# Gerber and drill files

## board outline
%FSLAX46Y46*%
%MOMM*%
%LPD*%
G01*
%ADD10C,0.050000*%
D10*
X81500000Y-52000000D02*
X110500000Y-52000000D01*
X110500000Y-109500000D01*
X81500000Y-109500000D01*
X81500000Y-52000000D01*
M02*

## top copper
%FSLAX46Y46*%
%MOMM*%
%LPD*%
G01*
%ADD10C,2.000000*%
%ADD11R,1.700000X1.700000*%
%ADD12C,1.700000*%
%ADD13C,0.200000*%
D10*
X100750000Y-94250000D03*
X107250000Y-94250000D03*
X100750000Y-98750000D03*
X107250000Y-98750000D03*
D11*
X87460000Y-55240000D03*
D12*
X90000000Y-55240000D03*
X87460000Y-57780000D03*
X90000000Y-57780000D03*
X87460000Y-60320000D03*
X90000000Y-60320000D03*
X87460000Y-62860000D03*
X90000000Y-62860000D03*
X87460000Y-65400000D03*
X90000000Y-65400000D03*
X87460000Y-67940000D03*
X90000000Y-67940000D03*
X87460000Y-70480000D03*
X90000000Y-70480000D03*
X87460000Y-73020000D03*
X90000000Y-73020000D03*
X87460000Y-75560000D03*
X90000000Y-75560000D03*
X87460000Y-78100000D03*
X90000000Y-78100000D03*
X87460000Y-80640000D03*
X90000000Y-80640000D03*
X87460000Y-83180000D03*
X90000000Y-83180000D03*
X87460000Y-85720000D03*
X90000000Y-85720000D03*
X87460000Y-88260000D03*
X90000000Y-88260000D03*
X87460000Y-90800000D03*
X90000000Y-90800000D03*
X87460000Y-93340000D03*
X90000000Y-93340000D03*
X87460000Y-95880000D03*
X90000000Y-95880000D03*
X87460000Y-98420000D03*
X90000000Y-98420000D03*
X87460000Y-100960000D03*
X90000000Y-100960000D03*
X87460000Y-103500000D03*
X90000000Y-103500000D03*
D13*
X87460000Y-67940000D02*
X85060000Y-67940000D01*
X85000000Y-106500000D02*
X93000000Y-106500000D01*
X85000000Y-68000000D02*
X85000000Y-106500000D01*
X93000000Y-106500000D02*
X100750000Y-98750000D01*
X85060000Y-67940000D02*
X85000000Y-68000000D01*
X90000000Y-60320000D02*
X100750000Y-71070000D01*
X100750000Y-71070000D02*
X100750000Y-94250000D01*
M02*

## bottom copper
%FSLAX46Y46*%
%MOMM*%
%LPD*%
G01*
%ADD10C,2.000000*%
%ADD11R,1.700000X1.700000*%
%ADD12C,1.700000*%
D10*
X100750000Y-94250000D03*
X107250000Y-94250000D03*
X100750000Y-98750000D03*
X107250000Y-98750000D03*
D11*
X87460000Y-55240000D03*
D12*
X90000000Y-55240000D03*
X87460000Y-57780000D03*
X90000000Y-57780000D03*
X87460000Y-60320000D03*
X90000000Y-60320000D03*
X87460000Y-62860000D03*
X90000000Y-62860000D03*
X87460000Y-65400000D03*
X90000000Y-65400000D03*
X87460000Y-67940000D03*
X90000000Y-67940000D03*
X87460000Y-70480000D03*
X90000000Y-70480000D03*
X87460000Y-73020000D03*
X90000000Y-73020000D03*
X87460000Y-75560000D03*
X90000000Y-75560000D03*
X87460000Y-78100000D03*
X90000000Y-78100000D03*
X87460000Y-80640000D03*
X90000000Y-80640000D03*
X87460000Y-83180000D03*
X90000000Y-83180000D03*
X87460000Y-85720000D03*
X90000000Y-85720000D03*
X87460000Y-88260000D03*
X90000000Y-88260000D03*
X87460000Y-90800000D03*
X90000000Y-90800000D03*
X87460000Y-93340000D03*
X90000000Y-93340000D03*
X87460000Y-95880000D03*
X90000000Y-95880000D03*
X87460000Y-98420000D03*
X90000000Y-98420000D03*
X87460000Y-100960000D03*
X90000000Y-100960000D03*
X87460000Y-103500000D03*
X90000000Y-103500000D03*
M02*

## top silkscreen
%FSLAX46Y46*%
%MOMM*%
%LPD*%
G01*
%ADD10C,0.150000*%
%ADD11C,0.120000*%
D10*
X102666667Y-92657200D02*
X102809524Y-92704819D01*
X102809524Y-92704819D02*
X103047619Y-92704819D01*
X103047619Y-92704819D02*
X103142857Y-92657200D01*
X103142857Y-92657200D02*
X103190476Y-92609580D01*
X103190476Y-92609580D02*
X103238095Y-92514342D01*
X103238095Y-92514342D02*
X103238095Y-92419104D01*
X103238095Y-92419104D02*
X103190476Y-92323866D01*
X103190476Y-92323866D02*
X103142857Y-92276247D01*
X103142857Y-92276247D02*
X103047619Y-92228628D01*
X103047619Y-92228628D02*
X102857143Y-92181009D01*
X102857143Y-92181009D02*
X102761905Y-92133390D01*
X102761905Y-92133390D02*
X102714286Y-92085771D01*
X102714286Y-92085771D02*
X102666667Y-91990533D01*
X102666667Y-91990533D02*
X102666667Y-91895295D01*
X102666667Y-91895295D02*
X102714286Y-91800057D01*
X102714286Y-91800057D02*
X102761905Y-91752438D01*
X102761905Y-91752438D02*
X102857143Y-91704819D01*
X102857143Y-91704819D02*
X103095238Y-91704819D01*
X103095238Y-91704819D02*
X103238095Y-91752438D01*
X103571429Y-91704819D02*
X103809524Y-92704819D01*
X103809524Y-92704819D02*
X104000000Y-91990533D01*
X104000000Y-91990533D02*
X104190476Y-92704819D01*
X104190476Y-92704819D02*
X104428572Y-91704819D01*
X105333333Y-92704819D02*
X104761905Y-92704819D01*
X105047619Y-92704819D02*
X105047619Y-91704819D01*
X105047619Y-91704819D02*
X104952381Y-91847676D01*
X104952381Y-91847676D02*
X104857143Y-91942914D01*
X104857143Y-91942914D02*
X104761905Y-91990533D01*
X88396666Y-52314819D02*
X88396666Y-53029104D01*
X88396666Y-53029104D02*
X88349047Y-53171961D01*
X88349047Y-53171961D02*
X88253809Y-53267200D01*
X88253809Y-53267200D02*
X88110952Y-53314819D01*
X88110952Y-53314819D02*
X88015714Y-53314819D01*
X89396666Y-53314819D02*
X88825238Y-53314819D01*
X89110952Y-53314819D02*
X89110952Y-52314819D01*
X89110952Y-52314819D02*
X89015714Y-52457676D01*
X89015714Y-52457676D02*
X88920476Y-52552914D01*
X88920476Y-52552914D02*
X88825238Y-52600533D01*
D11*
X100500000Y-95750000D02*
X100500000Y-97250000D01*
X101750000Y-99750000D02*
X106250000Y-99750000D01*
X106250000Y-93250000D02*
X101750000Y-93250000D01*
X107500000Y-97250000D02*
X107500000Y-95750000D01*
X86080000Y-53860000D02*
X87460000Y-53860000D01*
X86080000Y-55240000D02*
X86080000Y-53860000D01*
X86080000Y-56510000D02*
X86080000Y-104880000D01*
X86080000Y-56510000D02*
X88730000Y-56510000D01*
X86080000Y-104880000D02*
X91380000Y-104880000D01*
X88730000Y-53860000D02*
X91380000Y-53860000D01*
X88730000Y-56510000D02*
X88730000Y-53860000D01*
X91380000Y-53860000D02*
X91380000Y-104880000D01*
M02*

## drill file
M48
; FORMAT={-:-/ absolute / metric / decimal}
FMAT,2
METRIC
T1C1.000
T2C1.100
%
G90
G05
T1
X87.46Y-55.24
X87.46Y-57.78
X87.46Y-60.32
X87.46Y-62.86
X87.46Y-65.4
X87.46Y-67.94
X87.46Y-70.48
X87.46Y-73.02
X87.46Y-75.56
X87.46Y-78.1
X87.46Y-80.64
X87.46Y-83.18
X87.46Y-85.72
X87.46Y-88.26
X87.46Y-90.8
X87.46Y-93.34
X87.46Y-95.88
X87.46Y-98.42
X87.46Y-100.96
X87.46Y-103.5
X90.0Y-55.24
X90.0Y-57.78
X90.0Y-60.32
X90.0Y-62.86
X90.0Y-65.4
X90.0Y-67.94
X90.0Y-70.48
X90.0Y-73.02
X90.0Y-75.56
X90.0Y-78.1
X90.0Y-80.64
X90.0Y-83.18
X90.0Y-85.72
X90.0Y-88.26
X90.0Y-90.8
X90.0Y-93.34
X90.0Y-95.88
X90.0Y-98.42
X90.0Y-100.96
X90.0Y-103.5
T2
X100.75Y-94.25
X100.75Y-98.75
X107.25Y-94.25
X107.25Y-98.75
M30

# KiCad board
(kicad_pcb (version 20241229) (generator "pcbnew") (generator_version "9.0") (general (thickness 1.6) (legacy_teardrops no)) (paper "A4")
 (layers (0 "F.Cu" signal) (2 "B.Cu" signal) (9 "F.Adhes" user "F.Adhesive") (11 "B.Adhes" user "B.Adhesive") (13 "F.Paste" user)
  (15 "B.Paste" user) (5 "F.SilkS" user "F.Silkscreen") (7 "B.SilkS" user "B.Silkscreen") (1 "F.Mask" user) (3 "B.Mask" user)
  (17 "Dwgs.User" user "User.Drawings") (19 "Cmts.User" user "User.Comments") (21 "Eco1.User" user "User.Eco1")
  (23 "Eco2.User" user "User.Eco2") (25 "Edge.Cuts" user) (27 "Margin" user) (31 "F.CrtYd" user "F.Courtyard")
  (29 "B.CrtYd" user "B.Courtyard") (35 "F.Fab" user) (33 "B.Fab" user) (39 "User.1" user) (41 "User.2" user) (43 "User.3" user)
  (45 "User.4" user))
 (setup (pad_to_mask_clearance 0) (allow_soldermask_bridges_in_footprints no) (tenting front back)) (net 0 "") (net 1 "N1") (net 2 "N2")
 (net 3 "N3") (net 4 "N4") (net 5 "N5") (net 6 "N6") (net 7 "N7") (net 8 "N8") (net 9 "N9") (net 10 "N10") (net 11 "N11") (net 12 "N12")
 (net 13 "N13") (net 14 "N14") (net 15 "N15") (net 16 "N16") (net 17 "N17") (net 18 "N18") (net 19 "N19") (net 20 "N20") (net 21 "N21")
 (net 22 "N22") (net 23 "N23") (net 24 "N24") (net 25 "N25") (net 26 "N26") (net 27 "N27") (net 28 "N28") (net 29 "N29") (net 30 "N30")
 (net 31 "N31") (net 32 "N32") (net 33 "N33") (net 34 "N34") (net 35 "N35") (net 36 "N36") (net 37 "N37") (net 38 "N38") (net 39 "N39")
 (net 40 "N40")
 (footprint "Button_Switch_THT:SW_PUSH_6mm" (layer "F.Cu") (at 100.75 94.25)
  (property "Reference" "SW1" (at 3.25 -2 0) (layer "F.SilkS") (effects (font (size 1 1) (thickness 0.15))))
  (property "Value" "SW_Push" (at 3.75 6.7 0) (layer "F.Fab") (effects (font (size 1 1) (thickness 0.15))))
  (fp_line (start -0.25 1.5) (end -0.25 3) (stroke (width 0.12) (type solid)) (layer "F.SilkS"))
  (fp_line (start 1 5.5) (end 5.5 5.5) (stroke (width 0.12) (type solid)) (layer "F.SilkS"))
  (fp_line (start 5.5 -1) (end 1 -1) (stroke (width 0.12) (type solid)) (layer "F.SilkS"))
  (fp_line (start 6.75 3) (end 6.75 1.5) (stroke (width 0.12) (type solid)) (layer "F.SilkS"))
  (pad "1" thru_hole circle (at 0 0 90) (size 2 2) (drill 1.1) (layers "*.Cu" "*.Mask") (remove_unused_layers no) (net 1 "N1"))
  (pad "1" thru_hole circle (at 6.5 0 90) (size 2 2) (drill 1.1) (layers "*.Cu" "*.Mask") (remove_unused_layers no) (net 1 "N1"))
  (pad "2" thru_hole circle (at 0 4.5 90) (size 2 2) (drill 1.1) (layers "*.Cu" "*.Mask") (remove_unused_layers no) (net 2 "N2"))
  (pad "2" thru_hole circle (at 6.5 4.5 90) (size 2 2) (drill 1.1) (layers "*.Cu" "*.Mask") (remove_unused_layers no) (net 2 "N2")))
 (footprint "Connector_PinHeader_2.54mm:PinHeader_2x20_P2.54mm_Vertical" (layer "F.Cu") (at 87.46 55.24)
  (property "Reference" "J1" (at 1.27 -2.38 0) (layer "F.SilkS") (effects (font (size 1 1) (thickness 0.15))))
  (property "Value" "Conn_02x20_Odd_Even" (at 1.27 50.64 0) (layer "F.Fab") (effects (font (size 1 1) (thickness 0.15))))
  (fp_line (start -1.38 -1.38) (end 0 -1.38) (stroke (width 0.12) (type solid)) (layer "F.SilkS"))
  (fp_line (start -1.38 0) (end -1.38 -1.38) (stroke (width 0.12) (type solid)) (layer "F.SilkS"))
  (fp_line (start -1.38 1.27) (end -1.38 49.64) (stroke (width 0.12) (type solid)) (layer "F.SilkS"))
  (fp_line (start -1.38 1.27) (end 1.27 1.27) (stroke (width 0.12) (type solid)) (layer "F.SilkS"))
  (fp_line (start -1.38 49.64) (end 3.92 49.64) (stroke (width 0.12) (type solid)) (layer "F.SilkS"))
  (fp_line (start 1.27 -1.38) (end 3.92 -1.38) (stroke (width 0.12) (type solid)) (layer "F.SilkS"))
  (fp_line (start 1.27 1.27) (end 1.27 -1.38) (stroke (width 0.12) (type solid)) (layer "F.SilkS"))
  (fp_line (start 3.92 -1.38) (end 3.92 49.64) (stroke (width 0.12) (type solid)) (layer "F.SilkS"))
  (pad "1" thru_hole rect (at 0 0) (size 1.7 1.7) (drill 1) (layers "*.Cu" "*.Mask") (remove_unused_layers no) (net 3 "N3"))
  (pad "2" thru_hole circle (at 2.54 0) (size 1.7 1.7) (drill 1) (layers "*.Cu" "*.Mask") (remove_unused_layers no) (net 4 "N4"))
  (pad "3" thru_hole circle (at 0 2.54) (size 1.7 1.7) (drill 1) (layers "*.Cu" "*.Mask") (remove_unused_layers no) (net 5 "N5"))
  (pad "4" thru_hole circle (at 2.54 2.54) (size 1.7 1.7) (drill 1) (layers "*.Cu" "*.Mask") (remove_unused_layers no) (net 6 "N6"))
  (pad "5" thru_hole circle (at 0 5.08) (size 1.7 1.7) (drill 1) (layers "*.Cu" "*.Mask") (remove_unused_layers no) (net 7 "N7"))
  (pad "6" thru_hole circle (at 2.54 5.08) (size 1.7 1.7) (drill 1) (layers "*.Cu" "*.Mask") (remove_unused_layers no) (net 1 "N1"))
  (pad "7" thru_hole circle (at 0 7.62) (size 1.7 1.7) (drill 1) (layers "*.Cu" "*.Mask") (remove_unused_layers no) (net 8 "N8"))
  (pad "8" thru_hole circle (at 2.54 7.62) (size 1.7 1.7) (drill 1) (layers "*.Cu" "*.Mask") (remove_unused_layers no) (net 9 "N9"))
  (pad "9" thru_hole circle (at 0 10.16) (size 1.7 1.7) (drill 1) (layers "*.Cu" "*.Mask") (remove_unused_layers no) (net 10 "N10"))
  (pad "10" thru_hole circle (at 2.54 10.16) (size 1.7 1.7) (drill 1) (layers "*.Cu" "*.Mask") (remove_unused_layers no) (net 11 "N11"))
  (pad "11" thru_hole circle (at 0 12.7) (size 1.7 1.7) (drill 1) (layers "*.Cu" "*.Mask") (remove_unused_layers no) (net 2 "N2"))
  (pad "12" thru_hole circle (at 2.54 12.7) (size 1.7 1.7) (drill 1) (layers "*.Cu" "*.Mask") (remove_unused_layers no) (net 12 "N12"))
  (pad "13" thru_hole circle (at 0 15.24) (size 1.7 1.7) (drill 1) (layers "*.Cu" "*.Mask") (remove_unused_layers no) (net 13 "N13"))
  (pad "14" thru_hole circle (at 2.54 15.24) (size 1.7 1.7) (drill 1) (layers "*.Cu" "*.Mask") (remove_unused_layers no) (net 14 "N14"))
  (pad "15" thru_hole circle (at 0 17.78) (size 1.7 1.7) (drill 1) (layers "*.Cu" "*.Mask") (remove_unused_layers no) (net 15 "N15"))
  (pad "16" thru_hole circle (at 2.54 17.78) (size 1.7 1.7) (drill 1) (layers "*.Cu" "*.Mask") (remove_unused_layers no) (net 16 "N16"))
  (pad "17" thru_hole circle (at 0 20.32) (size 1.7 1.7) (drill 1) (layers "*.Cu" "*.Mask") (remove_unused_layers no) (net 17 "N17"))
  (pad "18" thru_hole circle (at 2.54 20.32) (size 1.7 1.7) (drill 1) (layers "*.Cu" "*.Mask") (remove_unused_layers no) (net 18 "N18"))
  (pad "19" thru_hole circle (at 0 22.86) (size 1.7 1.7) (drill 1) (layers "*.Cu" "*.Mask") (remove_unused_layers no) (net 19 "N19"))
  (pad "20" thru_hole circle (at 2.54 22.86) (size 1.7 1.7) (drill 1) (layers "*.Cu" "*.Mask") (remove_unused_layers no) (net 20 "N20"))
  (pad "21" thru_hole circle (at 0 25.4) (size 1.7 1.7) (drill 1) (layers "*.Cu" "*.Mask") (remove_unused_layers no) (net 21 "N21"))
  (pad "22" thru_hole circle (at 2.54 25.4) (size 1.7 1.7) (drill 1) (layers "*.Cu" "*.Mask") (remove_unused_layers no) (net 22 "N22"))
  (pad "23" thru_hole circle (at 0 27.94) (size 1.7 1.7) (drill 1) (layers "*.Cu" "*.Mask") (remove_unused_layers no) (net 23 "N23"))
  (pad "24" thru_hole circle (at 2.54 27.94) (size 1.7 1.7) (drill 1) (layers "*.Cu" "*.Mask") (remove_unused_layers no) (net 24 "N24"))
  (pad "25" thru_hole circle (at 0 30.48) (size 1.7 1.7) (drill 1) (layers "*.Cu" "*.Mask") (remove_unused_layers no) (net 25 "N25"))
  (pad "26" thru_hole circle (at 2.54 30.48) (size 1.7 1.7) (drill 1) (layers "*.Cu" "*.Mask") (remove_unused_layers no) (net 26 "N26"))
  (pad "27" thru_hole circle (at 0 33.02) (size 1.7 1.7) (drill 1) (layers "*.Cu" "*.Mask") (remove_unused_layers no) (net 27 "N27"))
  (pad "28" thru_hole circle (at 2.54 33.02) (size 1.7 1.7) (drill 1) (layers "*.Cu" "*.Mask") (remove_unused_layers no) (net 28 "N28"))
  (pad "29" thru_hole circle (at 0 35.56) (size 1.7 1.7) (drill 1) (layers "*.Cu" "*.Mask") (remove_unused_layers no) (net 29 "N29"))
  (pad "30" thru_hole circle (at 2.54 35.56) (size 1.7 1.7) (drill 1) (layers "*.Cu" "*.Mask") (remove_unused_layers no) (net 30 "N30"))
  (pad "31" thru_hole circle (at 0 38.1) (size 1.7 1.7) (drill 1) (layers "*.Cu" "*.Mask") (remove_unused_layers no) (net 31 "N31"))
  (pad "32" thru_hole circle (at 2.54 38.1) (size 1.7 1.7) (drill 1) (layers "*.Cu" "*.Mask") (remove_unused_layers no) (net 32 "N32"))
  (pad "33" thru_hole circle (at 0 40.64) (size 1.7 1.7) (drill 1) (layers "*.Cu" "*.Mask") (remove_unused_layers no) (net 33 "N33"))
  (pad "34" thru_hole circle (at 2.54 40.64) (size 1.7 1.7) (drill 1) (layers "*.Cu" "*.Mask") (remove_unused_layers no) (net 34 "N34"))
  (pad "35" thru_hole circle (at 0 43.18) (size 1.7 1.7) (drill 1) (layers "*.Cu" "*.Mask") (remove_unused_layers no) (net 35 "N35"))
  (pad "36" thru_hole circle (at 2.54 43.18) (size 1.7 1.7) (drill 1) (layers "*.Cu" "*.Mask") (remove_unused_layers no) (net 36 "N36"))
  (pad "37" thru_hole circle (at 0 45.72) (size 1.7 1.7) (drill 1) (layers "*.Cu" "*.Mask") (remove_unused_layers no) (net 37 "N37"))
  (pad "38" thru_hole circle (at 2.54 45.72) (size 1.7 1.7) (drill 1) (layers "*.Cu" "*.Mask") (remove_unused_layers no) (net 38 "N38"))
  (pad "39" thru_hole circle (at 0 48.26) (size 1.7 1.7) (drill 1) (layers "*.Cu" "*.Mask") (remove_unused_layers no) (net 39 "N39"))
  (pad "40" thru_hole circle (at 2.54 48.26) (size 1.7 1.7) (drill 1) (layers "*.Cu" "*.Mask") (remove_unused_layers no) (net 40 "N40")))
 (gr_rect (start 81.5 52) (end 110.5 109.5) (stroke (width 0.05) (type default)) (fill no) (layer "Edge.Cuts"))
 (segment (start 87.46 67.94) (end 85.06 67.94) (width 0.2) (layer "F.Cu") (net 2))
 (segment (start 85 106.5) (end 93 106.5) (width 0.2) (layer "F.Cu") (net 2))
 (segment (start 85 68) (end 85 106.5) (width 0.2) (layer "F.Cu") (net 2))
 (segment (start 93 106.5) (end 100.75 98.75) (width 0.2) (layer "F.Cu") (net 2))
 (segment (start 85.06 67.94) (end 85 68) (width 0.2) (layer "F.Cu") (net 2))
 (segment (start 90 60.32) (end 100.75 71.07) (width 0.2) (layer "F.Cu") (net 1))
 (segment (start 100.75 71.07) (end 100.75 94.25) (width 0.2) (layer "F.Cu") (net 1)))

